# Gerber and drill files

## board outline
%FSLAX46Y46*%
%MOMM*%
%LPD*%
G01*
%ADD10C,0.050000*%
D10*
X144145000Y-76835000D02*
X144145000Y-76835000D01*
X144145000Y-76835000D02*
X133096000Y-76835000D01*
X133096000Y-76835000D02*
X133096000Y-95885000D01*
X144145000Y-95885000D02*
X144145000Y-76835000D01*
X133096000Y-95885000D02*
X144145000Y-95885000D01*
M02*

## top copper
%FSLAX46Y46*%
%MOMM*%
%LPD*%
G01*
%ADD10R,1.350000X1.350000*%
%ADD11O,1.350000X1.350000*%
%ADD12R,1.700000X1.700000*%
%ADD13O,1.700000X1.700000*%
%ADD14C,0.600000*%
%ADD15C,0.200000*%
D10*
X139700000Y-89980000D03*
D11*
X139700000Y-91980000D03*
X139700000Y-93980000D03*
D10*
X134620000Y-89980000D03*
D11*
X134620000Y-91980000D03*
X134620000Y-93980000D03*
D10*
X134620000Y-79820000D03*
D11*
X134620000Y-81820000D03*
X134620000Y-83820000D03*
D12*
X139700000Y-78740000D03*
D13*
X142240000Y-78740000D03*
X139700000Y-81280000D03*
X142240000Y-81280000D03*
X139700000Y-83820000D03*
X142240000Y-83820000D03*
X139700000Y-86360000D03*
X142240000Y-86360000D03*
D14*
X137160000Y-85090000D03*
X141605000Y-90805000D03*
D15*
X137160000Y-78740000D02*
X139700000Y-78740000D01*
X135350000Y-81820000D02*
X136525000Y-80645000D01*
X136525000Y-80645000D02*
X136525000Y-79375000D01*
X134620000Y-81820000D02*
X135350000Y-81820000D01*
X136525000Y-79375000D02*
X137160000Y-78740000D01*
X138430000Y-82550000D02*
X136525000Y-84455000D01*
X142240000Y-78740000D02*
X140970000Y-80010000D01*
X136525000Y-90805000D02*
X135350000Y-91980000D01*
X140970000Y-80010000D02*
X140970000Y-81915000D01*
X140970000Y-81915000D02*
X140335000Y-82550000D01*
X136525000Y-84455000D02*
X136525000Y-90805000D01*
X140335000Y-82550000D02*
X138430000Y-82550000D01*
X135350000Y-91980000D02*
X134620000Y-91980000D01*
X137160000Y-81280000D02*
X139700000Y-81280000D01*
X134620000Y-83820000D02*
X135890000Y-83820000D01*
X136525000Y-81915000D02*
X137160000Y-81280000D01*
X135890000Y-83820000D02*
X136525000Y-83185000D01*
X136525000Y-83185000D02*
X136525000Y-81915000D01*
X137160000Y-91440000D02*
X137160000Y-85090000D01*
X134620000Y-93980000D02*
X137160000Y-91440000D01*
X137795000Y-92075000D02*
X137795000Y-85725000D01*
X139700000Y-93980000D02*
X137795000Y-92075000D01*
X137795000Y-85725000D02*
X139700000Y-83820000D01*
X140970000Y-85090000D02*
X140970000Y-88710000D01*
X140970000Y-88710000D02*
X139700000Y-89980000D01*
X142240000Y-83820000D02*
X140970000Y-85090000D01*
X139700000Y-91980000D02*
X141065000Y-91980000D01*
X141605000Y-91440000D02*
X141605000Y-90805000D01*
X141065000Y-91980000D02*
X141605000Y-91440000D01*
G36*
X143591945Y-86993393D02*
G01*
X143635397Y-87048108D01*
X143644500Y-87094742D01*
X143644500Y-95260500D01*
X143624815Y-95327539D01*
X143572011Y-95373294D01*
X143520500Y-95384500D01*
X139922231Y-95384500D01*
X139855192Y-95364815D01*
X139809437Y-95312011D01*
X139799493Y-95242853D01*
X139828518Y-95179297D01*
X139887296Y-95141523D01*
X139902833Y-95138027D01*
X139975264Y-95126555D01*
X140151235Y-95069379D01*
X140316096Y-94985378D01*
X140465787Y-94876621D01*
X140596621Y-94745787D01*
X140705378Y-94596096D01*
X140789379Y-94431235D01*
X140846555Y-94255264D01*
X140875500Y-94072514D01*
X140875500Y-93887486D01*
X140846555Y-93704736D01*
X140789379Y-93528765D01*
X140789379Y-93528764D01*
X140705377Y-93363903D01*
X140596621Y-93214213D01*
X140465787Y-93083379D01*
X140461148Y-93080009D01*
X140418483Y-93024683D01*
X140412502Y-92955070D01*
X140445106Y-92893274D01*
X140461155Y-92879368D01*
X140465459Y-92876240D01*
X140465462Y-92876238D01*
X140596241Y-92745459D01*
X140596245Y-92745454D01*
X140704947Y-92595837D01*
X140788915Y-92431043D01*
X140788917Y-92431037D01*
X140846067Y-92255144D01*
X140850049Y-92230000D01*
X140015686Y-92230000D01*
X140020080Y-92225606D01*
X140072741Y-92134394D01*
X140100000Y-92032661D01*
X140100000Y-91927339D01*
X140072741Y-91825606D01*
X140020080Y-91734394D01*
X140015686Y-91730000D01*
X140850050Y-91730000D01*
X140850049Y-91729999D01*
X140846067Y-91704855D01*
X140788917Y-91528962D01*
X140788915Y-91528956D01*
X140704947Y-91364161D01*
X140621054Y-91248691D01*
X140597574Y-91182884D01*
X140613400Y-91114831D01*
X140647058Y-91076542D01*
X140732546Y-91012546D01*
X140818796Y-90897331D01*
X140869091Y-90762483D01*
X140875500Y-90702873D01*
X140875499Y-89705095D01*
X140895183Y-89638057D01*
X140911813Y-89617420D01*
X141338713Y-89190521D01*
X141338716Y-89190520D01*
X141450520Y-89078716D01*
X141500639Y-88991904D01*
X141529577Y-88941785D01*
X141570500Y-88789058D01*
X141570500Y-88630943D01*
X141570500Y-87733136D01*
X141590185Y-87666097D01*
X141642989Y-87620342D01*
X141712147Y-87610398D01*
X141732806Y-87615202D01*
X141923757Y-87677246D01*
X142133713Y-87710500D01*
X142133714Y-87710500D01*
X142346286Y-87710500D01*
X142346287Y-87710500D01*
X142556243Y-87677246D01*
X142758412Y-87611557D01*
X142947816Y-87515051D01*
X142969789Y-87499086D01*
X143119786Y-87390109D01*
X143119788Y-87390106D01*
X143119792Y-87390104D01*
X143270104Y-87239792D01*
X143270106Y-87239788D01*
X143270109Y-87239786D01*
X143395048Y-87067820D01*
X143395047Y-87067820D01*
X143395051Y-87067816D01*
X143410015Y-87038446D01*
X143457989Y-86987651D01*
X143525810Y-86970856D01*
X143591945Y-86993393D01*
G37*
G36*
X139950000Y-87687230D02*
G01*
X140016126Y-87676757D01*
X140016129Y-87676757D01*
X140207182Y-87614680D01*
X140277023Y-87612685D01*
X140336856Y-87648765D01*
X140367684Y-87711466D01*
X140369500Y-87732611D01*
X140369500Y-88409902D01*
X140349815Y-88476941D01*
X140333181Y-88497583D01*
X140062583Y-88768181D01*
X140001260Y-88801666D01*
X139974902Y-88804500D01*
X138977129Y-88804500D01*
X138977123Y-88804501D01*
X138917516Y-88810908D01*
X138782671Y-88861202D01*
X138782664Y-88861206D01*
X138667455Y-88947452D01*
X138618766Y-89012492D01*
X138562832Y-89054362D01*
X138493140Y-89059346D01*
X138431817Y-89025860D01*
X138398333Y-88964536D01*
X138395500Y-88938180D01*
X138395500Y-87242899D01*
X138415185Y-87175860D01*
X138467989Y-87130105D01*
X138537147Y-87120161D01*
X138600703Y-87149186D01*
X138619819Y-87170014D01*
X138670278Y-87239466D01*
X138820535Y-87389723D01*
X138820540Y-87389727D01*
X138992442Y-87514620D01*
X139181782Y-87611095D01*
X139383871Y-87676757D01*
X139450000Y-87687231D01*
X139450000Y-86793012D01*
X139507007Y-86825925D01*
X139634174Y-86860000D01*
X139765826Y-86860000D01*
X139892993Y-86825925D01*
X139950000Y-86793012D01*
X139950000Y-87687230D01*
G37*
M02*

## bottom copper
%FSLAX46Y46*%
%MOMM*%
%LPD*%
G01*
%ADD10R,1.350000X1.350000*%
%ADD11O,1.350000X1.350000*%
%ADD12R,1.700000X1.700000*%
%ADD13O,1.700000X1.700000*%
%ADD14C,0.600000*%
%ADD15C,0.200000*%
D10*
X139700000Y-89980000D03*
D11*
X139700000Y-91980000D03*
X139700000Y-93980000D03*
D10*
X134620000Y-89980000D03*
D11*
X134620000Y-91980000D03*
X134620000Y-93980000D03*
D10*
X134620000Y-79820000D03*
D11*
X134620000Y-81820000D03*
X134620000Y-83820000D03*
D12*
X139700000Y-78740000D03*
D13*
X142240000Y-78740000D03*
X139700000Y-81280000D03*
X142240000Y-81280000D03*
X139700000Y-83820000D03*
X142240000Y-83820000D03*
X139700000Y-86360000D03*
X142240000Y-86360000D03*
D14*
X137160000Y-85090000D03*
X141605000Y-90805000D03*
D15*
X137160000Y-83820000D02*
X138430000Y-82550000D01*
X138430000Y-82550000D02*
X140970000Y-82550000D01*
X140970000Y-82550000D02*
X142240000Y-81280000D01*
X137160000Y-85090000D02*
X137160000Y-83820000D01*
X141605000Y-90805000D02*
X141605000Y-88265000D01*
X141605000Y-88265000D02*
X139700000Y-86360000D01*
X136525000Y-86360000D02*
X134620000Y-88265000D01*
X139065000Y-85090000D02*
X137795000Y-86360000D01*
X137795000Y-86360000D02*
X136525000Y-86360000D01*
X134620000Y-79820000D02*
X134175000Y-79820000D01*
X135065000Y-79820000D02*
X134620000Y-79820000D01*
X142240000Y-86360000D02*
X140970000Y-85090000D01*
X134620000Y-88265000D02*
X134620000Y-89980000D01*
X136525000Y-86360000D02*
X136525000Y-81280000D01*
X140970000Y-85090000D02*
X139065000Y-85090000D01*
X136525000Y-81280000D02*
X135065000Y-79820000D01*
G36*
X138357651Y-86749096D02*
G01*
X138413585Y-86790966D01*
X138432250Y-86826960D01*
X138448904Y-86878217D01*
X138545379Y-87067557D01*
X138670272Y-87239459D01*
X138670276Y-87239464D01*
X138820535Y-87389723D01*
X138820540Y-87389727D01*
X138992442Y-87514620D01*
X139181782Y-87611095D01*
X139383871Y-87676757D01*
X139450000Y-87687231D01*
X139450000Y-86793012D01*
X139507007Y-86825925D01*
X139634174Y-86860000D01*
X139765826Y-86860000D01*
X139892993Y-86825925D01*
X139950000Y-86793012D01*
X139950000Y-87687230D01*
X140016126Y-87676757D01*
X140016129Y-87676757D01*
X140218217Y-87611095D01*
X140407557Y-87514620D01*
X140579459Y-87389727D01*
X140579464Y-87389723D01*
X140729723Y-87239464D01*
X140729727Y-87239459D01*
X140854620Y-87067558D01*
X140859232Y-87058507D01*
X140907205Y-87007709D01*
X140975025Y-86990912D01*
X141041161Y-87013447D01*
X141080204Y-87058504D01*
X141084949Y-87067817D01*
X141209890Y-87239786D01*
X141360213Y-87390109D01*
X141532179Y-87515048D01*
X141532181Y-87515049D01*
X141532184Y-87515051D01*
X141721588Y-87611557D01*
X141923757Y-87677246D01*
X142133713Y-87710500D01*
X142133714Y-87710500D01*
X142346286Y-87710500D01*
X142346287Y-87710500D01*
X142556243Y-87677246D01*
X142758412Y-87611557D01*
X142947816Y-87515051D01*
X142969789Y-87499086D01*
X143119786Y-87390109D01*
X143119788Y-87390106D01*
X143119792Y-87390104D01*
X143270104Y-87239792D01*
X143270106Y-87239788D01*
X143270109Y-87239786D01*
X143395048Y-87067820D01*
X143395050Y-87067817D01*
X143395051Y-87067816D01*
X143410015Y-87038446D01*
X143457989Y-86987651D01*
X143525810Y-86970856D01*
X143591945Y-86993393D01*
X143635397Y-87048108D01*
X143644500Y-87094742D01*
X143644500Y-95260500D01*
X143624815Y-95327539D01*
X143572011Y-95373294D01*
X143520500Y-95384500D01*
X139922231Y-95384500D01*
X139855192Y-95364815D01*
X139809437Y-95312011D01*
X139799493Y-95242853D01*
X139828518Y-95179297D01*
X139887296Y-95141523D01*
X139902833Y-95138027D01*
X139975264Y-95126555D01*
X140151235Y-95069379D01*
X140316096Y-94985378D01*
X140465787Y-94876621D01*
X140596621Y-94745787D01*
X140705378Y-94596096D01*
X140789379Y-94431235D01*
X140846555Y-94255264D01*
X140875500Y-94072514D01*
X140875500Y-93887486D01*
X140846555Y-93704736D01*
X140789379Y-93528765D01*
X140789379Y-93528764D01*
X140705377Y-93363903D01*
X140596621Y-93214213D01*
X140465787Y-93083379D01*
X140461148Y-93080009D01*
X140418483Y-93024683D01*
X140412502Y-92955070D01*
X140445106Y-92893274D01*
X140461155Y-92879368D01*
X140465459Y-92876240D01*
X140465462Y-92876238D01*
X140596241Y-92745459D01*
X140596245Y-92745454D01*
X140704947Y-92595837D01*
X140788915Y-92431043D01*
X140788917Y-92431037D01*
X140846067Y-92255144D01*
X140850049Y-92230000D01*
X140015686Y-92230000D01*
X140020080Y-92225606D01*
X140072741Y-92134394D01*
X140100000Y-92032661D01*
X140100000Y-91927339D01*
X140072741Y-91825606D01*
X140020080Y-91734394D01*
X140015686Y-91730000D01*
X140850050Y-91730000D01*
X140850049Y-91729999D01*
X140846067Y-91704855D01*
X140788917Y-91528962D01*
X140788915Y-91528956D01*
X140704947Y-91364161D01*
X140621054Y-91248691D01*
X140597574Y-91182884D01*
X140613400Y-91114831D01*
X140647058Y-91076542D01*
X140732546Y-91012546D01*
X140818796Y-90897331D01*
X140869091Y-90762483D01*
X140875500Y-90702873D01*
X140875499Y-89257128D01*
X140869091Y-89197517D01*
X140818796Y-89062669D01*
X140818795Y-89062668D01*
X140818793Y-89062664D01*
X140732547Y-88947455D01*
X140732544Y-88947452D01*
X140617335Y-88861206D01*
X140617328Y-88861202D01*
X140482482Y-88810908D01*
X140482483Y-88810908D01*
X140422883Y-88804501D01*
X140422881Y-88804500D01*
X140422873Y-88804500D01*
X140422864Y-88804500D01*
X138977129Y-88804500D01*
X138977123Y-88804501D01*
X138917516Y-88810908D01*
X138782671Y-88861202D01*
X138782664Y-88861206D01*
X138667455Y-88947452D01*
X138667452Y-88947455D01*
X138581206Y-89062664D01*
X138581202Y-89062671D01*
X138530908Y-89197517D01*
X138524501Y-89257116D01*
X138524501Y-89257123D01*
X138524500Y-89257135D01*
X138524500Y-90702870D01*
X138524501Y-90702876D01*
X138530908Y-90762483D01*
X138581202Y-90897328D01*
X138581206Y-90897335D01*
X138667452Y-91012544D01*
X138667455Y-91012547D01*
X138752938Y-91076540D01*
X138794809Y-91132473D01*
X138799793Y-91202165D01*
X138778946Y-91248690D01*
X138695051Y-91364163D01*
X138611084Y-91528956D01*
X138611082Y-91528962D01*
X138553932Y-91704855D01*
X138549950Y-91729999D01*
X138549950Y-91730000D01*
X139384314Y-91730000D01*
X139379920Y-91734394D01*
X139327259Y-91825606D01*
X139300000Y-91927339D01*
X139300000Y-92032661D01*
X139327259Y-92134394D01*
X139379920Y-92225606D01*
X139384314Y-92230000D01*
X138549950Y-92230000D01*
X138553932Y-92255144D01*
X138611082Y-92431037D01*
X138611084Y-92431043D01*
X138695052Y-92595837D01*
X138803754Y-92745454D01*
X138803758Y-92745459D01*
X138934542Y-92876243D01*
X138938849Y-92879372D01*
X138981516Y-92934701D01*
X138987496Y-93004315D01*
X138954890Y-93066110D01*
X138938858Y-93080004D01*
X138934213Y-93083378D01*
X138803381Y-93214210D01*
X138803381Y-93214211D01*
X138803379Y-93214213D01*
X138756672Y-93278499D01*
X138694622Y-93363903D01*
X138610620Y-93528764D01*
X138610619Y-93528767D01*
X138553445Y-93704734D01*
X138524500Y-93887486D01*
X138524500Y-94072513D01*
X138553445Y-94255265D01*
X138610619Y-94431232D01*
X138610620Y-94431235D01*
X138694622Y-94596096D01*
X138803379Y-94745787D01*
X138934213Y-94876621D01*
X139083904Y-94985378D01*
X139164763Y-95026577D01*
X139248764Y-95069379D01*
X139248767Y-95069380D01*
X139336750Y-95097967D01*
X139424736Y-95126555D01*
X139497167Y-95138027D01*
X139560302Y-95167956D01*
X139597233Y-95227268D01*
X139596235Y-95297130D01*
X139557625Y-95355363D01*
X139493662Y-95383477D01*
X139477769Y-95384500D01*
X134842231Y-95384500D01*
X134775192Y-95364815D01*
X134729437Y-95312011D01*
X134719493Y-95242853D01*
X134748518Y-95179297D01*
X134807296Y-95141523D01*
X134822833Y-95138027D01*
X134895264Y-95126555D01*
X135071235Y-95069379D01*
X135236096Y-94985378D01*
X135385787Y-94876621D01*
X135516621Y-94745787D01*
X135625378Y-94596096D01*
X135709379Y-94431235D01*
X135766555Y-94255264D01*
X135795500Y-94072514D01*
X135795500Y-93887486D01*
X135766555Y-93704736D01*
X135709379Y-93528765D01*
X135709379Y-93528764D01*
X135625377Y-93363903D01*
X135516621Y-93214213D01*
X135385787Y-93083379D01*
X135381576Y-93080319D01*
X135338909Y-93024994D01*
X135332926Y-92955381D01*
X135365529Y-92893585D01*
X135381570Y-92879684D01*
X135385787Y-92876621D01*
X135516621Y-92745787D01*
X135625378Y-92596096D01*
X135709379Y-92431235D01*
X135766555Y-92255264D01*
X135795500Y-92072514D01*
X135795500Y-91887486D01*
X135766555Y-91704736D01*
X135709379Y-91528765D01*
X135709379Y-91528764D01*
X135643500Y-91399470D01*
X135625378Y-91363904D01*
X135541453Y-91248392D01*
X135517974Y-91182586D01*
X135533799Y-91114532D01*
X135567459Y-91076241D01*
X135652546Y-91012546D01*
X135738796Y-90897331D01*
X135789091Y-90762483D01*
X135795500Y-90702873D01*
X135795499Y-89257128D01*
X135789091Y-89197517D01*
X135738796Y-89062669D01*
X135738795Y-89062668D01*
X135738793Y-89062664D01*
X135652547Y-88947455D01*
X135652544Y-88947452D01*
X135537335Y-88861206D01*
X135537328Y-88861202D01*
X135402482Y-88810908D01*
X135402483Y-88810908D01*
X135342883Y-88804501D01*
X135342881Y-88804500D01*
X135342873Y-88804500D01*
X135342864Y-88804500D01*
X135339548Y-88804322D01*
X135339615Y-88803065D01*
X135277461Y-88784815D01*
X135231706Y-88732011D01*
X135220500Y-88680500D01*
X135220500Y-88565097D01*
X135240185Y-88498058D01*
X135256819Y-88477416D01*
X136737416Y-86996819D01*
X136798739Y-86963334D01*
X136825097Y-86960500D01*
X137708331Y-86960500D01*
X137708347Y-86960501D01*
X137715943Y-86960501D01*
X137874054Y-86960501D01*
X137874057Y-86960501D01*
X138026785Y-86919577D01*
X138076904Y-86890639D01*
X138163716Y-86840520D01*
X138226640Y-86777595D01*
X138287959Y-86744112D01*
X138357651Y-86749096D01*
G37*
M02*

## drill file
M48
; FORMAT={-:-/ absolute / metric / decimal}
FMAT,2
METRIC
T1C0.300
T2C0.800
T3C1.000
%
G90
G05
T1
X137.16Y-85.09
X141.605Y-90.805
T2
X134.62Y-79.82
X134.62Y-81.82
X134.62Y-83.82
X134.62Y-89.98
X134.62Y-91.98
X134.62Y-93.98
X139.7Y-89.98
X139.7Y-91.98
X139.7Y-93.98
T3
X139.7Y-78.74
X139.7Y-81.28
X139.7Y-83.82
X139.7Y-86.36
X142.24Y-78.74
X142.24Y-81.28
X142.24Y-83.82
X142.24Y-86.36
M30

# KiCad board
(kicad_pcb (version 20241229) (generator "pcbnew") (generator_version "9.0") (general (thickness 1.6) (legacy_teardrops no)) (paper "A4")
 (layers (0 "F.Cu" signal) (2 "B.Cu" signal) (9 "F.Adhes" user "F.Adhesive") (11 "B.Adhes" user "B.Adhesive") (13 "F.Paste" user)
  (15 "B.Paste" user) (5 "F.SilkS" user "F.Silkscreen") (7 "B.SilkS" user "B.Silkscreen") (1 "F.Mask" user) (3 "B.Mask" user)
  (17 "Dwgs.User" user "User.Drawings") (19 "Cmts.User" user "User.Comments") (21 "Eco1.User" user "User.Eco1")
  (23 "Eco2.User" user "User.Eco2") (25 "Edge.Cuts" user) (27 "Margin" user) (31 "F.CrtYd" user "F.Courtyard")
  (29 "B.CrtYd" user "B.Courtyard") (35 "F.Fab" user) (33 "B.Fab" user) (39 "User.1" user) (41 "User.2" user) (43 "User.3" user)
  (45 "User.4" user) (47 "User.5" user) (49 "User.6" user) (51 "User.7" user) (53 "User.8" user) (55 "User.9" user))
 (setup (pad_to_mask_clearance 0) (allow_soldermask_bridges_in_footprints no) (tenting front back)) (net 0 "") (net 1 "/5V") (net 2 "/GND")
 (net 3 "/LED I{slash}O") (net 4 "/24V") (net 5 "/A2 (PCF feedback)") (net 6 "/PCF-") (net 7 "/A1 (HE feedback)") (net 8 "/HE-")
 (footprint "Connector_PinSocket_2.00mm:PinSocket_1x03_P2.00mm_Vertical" (layer "F.Cu") (at 139.7 89.98)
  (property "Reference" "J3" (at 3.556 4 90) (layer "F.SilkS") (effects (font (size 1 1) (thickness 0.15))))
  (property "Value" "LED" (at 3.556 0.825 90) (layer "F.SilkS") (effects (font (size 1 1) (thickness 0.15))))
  (pad "1" thru_hole rect (at 0 0) (size 1.35 1.35) (drill 0.8) (layers "*.Cu" "*.Mask") (remove_unused_layers no) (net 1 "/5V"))
  (pad "2" thru_hole oval (at 0 2) (size 1.35 1.35) (drill 0.8) (layers "*.Cu" "*.Mask") (remove_unused_layers no) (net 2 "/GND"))
  (pad "3" thru_hole oval (at 0 4) (size 1.35 1.35) (drill 0.8) (layers "*.Cu" "*.Mask") (remove_unused_layers no) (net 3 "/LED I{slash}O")))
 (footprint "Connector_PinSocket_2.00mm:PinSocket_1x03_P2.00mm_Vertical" (layer "F.Cu") (at 134.62 89.98)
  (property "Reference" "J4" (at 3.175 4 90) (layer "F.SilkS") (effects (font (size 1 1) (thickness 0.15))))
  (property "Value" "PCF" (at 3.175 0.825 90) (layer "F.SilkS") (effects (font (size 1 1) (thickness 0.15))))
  (pad "1" thru_hole rect (at 0 0) (size 1.35 1.35) (drill 0.8) (layers "*.Cu" "*.Mask") (remove_unused_layers no) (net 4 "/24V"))
  (pad "2" thru_hole oval (at 0 2) (size 1.35 1.35) (drill 0.8) (layers "*.Cu" "*.Mask") (remove_unused_layers no)
   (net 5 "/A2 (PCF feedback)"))
  (pad "3" thru_hole oval (at 0 4) (size 1.35 1.35) (drill 0.8) (layers "*.Cu" "*.Mask") (remove_unused_layers no) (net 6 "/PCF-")))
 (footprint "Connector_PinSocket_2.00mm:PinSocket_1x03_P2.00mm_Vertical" (layer "F.Cu") (at 134.62 79.82)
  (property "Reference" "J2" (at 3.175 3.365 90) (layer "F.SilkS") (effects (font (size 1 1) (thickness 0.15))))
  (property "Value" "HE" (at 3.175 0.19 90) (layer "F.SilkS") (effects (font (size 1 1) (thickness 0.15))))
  (pad "1" thru_hole rect (at 0 0) (size 1.35 1.35) (drill 0.8) (layers "*.Cu" "*.Mask") (remove_unused_layers no) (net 4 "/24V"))
  (pad "2" thru_hole oval (at 0 2) (size 1.35 1.35) (drill 0.8) (layers "*.Cu" "*.Mask") (remove_unused_layers no)
   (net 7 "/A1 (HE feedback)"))
  (pad "3" thru_hole oval (at 0 4) (size 1.35 1.35) (drill 0.8) (layers "*.Cu" "*.Mask") (remove_unused_layers no) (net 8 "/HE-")))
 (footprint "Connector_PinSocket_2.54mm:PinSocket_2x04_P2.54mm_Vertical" (layer "B.Cu") (at 139.7 78.74 180)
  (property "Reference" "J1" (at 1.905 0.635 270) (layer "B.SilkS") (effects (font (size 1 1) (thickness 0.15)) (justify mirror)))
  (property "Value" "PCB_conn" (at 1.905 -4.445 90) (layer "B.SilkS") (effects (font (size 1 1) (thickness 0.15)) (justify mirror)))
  (pad "1" thru_hole rect (at 0 0 180) (size 1.7 1.7) (drill 1) (layers "*.Cu" "*.Mask") (remove_unused_layers no)
   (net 7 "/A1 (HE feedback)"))
  (pad "2" thru_hole oval (at -2.54 0 180) (size 1.7 1.7) (drill 1) (layers "*.Cu" "*.Mask") (remove_unused_layers no)
   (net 5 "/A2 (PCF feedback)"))
  (pad "3" thru_hole oval (at 0 -2.54 180) (size 1.7 1.7) (drill 1) (layers "*.Cu" "*.Mask") (remove_unused_layers no) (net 8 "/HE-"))
  (pad "4" thru_hole oval (at -2.54 -2.54 180) (size 1.7 1.7) (drill 1) (layers "*.Cu" "*.Mask") (remove_unused_layers no) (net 6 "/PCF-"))
  (pad "5" thru_hole oval (at 0 -5.08 180) (size 1.7 1.7) (drill 1) (layers "*.Cu" "*.Mask") (remove_unused_layers no)
   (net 3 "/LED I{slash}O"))
  (pad "6" thru_hole oval (at -2.54 -5.08 180) (size 1.7 1.7) (drill 1) (layers "*.Cu" "*.Mask") (remove_unused_layers no) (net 1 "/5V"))
  (pad "7" thru_hole oval (at 0 -7.62 180) (size 1.7 1.7) (drill 1) (layers "*.Cu" "*.Mask") (remove_unused_layers no) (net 2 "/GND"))
  (pad "8" thru_hole oval (at -2.54 -7.62 180) (size 1.7 1.7) (drill 1) (layers "*.Cu" "*.Mask") (remove_unused_layers no) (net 4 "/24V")))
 (gr_line (start 144.145 76.835) (end 144.145 76.835) (stroke (width 0.05) (type default)) (layer "Edge.Cuts"))
 (gr_line (start 144.145 76.835) (end 133.096 76.835) (stroke (width 0.05) (type default)) (layer "Edge.Cuts"))
 (gr_line (start 133.096 76.835) (end 133.096 95.885) (stroke (width 0.05) (type default)) (layer "Edge.Cuts"))
 (gr_line (start 144.145 95.885) (end 144.145 76.835) (stroke (width 0.05) (type default)) (layer "Edge.Cuts"))
 (gr_line (start 133.096 95.885) (end 144.145 95.885) (stroke (width 0.05) (type default)) (layer "Edge.Cuts"))
 (segment (start 137.16 78.74) (end 139.7 78.74) (width 0.2) (layer "F.Cu") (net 7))
 (segment (start 135.35 81.82) (end 136.525 80.645) (width 0.2) (layer "F.Cu") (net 7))
 (segment (start 136.525 80.645) (end 136.525 79.375) (width 0.2) (layer "F.Cu") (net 7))
 (segment (start 134.62 81.82) (end 135.35 81.82) (width 0.2) (layer "F.Cu") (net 7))
 (segment (start 136.525 79.375) (end 137.16 78.74) (width 0.2) (layer "F.Cu") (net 7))
 (segment (start 138.43 82.55) (end 136.525 84.455) (width 0.2) (layer "F.Cu") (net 5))
 (segment (start 142.24 78.74) (end 140.97 80.01) (width 0.2) (layer "F.Cu") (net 5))
 (segment (start 136.525 90.805) (end 135.35 91.98) (width 0.2) (layer "F.Cu") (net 5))
 (segment (start 140.97 80.01) (end 140.97 81.915) (width 0.2) (layer "F.Cu") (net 5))
 (segment (start 140.97 81.915) (end 140.335 82.55) (width 0.2) (layer "F.Cu") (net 5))
 (segment (start 136.525 84.455) (end 136.525 90.805) (width 0.2) (layer "F.Cu") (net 5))
 (segment (start 140.335 82.55) (end 138.43 82.55) (width 0.2) (layer "F.Cu") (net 5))
 (segment (start 135.35 91.98) (end 134.62 91.98) (width 0.2) (layer "F.Cu") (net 5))
 (segment (start 137.16 81.28) (end 139.7 81.28) (width 0.2) (layer "F.Cu") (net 8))
 (segment (start 134.62 83.82) (end 135.89 83.82) (width 0.2) (layer "F.Cu") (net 8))
 (segment (start 136.525 81.915) (end 137.16 81.28) (width 0.2) (layer "F.Cu") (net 8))
 (segment (start 135.89 83.82) (end 136.525 83.185) (width 0.2) (layer "F.Cu") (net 8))
 (segment (start 136.525 83.185) (end 136.525 81.915) (width 0.2) (layer "F.Cu") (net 8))
 (segment (start 137.16 91.44) (end 137.16 85.09) (width 0.2) (layer "F.Cu") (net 6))
 (segment (start 134.62 93.98) (end 137.16 91.44) (width 0.2) (layer "F.Cu") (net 6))
 (via (at 137.16 85.09) (size 0.6) (drill 0.3) (layers "F.Cu" "B.Cu") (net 6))
 (segment (start 137.16 83.82) (end 138.43 82.55) (width 0.2) (layer "B.Cu") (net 6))
 (segment (start 138.43 82.55) (end 140.97 82.55) (width 0.2) (layer "B.Cu") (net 6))
 (segment (start 140.97 82.55) (end 142.24 81.28) (width 0.2) (layer "B.Cu") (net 6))
 (segment (start 137.16 85.09) (end 137.16 83.82) (width 0.2) (layer "B.Cu") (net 6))
 (segment (start 137.795 92.075) (end 137.795 85.725) (width 0.2) (layer "F.Cu") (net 3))
 (segment (start 139.7 93.98) (end 137.795 92.075) (width 0.2) (layer "F.Cu") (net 3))
 (segment (start 137.795 85.725) (end 139.7 83.82) (width 0.2) (layer "F.Cu") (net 3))
 (segment (start 140.97 85.09) (end 140.97 88.71) (width 0.2) (layer "F.Cu") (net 1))
 (segment (start 140.97 88.71) (end 139.7 89.98) (width 0.2) (layer "F.Cu") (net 1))
 (segment (start 142.24 83.82) (end 140.97 85.09) (width 0.2) (layer "F.Cu") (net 1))
 (segment (start 139.7 91.98) (end 141.065 91.98) (width 0.2) (layer "F.Cu") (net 2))
 (segment (start 141.605 91.44) (end 141.605 90.805) (width 0.2) (layer "F.Cu") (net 2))
 (segment (start 141.065 91.98) (end 141.605 91.44) (width 0.2) (layer "F.Cu") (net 2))
 (via (at 141.605 90.805) (size 0.6) (drill 0.3) (layers "F.Cu" "B.Cu") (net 2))
 (segment (start 141.605 90.805) (end 141.605 88.265) (width 0.2) (layer "B.Cu") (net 2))
 (segment (start 141.605 88.265) (end 139.7 86.36) (width 0.2) (layer "B.Cu") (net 2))
 (segment (start 136.525 86.36) (end 134.62 88.265) (width 0.2) (layer "B.Cu") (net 4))
 (segment (start 139.065 85.09) (end 137.795 86.36) (width 0.2) (layer "B.Cu") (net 4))
 (segment (start 137.795 86.36) (end 136.525 86.36) (width 0.2) (layer "B.Cu") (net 4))
 (segment (start 134.62 79.82) (end 134.175 79.82) (width 0.2) (layer "B.Cu") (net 4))
 (segment (start 135.065 79.82) (end 134.62 79.82) (width 0.2) (layer "B.Cu") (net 4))
 (segment (start 142.24 86.36) (end 140.97 85.09) (width 0.2) (layer "B.Cu") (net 4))
 (segment (start 134.62 88.265) (end 134.62 89.98) (width 0.2) (layer "B.Cu") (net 4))
 (segment (start 136.525 86.36) (end 136.525 81.28) (width 0.2) (layer "B.Cu") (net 4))
 (segment (start 140.97 85.09) (end 139.065 85.09) (width 0.2) (layer "B.Cu") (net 4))
 (segment (start 136.525 81.28) (end 135.065 79.82) (width 0.2) (layer "B.Cu") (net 4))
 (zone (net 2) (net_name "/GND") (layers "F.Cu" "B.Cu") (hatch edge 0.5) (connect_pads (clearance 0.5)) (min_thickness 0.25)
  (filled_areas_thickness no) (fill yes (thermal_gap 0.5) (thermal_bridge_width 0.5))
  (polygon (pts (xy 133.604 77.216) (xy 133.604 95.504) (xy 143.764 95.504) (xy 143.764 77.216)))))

